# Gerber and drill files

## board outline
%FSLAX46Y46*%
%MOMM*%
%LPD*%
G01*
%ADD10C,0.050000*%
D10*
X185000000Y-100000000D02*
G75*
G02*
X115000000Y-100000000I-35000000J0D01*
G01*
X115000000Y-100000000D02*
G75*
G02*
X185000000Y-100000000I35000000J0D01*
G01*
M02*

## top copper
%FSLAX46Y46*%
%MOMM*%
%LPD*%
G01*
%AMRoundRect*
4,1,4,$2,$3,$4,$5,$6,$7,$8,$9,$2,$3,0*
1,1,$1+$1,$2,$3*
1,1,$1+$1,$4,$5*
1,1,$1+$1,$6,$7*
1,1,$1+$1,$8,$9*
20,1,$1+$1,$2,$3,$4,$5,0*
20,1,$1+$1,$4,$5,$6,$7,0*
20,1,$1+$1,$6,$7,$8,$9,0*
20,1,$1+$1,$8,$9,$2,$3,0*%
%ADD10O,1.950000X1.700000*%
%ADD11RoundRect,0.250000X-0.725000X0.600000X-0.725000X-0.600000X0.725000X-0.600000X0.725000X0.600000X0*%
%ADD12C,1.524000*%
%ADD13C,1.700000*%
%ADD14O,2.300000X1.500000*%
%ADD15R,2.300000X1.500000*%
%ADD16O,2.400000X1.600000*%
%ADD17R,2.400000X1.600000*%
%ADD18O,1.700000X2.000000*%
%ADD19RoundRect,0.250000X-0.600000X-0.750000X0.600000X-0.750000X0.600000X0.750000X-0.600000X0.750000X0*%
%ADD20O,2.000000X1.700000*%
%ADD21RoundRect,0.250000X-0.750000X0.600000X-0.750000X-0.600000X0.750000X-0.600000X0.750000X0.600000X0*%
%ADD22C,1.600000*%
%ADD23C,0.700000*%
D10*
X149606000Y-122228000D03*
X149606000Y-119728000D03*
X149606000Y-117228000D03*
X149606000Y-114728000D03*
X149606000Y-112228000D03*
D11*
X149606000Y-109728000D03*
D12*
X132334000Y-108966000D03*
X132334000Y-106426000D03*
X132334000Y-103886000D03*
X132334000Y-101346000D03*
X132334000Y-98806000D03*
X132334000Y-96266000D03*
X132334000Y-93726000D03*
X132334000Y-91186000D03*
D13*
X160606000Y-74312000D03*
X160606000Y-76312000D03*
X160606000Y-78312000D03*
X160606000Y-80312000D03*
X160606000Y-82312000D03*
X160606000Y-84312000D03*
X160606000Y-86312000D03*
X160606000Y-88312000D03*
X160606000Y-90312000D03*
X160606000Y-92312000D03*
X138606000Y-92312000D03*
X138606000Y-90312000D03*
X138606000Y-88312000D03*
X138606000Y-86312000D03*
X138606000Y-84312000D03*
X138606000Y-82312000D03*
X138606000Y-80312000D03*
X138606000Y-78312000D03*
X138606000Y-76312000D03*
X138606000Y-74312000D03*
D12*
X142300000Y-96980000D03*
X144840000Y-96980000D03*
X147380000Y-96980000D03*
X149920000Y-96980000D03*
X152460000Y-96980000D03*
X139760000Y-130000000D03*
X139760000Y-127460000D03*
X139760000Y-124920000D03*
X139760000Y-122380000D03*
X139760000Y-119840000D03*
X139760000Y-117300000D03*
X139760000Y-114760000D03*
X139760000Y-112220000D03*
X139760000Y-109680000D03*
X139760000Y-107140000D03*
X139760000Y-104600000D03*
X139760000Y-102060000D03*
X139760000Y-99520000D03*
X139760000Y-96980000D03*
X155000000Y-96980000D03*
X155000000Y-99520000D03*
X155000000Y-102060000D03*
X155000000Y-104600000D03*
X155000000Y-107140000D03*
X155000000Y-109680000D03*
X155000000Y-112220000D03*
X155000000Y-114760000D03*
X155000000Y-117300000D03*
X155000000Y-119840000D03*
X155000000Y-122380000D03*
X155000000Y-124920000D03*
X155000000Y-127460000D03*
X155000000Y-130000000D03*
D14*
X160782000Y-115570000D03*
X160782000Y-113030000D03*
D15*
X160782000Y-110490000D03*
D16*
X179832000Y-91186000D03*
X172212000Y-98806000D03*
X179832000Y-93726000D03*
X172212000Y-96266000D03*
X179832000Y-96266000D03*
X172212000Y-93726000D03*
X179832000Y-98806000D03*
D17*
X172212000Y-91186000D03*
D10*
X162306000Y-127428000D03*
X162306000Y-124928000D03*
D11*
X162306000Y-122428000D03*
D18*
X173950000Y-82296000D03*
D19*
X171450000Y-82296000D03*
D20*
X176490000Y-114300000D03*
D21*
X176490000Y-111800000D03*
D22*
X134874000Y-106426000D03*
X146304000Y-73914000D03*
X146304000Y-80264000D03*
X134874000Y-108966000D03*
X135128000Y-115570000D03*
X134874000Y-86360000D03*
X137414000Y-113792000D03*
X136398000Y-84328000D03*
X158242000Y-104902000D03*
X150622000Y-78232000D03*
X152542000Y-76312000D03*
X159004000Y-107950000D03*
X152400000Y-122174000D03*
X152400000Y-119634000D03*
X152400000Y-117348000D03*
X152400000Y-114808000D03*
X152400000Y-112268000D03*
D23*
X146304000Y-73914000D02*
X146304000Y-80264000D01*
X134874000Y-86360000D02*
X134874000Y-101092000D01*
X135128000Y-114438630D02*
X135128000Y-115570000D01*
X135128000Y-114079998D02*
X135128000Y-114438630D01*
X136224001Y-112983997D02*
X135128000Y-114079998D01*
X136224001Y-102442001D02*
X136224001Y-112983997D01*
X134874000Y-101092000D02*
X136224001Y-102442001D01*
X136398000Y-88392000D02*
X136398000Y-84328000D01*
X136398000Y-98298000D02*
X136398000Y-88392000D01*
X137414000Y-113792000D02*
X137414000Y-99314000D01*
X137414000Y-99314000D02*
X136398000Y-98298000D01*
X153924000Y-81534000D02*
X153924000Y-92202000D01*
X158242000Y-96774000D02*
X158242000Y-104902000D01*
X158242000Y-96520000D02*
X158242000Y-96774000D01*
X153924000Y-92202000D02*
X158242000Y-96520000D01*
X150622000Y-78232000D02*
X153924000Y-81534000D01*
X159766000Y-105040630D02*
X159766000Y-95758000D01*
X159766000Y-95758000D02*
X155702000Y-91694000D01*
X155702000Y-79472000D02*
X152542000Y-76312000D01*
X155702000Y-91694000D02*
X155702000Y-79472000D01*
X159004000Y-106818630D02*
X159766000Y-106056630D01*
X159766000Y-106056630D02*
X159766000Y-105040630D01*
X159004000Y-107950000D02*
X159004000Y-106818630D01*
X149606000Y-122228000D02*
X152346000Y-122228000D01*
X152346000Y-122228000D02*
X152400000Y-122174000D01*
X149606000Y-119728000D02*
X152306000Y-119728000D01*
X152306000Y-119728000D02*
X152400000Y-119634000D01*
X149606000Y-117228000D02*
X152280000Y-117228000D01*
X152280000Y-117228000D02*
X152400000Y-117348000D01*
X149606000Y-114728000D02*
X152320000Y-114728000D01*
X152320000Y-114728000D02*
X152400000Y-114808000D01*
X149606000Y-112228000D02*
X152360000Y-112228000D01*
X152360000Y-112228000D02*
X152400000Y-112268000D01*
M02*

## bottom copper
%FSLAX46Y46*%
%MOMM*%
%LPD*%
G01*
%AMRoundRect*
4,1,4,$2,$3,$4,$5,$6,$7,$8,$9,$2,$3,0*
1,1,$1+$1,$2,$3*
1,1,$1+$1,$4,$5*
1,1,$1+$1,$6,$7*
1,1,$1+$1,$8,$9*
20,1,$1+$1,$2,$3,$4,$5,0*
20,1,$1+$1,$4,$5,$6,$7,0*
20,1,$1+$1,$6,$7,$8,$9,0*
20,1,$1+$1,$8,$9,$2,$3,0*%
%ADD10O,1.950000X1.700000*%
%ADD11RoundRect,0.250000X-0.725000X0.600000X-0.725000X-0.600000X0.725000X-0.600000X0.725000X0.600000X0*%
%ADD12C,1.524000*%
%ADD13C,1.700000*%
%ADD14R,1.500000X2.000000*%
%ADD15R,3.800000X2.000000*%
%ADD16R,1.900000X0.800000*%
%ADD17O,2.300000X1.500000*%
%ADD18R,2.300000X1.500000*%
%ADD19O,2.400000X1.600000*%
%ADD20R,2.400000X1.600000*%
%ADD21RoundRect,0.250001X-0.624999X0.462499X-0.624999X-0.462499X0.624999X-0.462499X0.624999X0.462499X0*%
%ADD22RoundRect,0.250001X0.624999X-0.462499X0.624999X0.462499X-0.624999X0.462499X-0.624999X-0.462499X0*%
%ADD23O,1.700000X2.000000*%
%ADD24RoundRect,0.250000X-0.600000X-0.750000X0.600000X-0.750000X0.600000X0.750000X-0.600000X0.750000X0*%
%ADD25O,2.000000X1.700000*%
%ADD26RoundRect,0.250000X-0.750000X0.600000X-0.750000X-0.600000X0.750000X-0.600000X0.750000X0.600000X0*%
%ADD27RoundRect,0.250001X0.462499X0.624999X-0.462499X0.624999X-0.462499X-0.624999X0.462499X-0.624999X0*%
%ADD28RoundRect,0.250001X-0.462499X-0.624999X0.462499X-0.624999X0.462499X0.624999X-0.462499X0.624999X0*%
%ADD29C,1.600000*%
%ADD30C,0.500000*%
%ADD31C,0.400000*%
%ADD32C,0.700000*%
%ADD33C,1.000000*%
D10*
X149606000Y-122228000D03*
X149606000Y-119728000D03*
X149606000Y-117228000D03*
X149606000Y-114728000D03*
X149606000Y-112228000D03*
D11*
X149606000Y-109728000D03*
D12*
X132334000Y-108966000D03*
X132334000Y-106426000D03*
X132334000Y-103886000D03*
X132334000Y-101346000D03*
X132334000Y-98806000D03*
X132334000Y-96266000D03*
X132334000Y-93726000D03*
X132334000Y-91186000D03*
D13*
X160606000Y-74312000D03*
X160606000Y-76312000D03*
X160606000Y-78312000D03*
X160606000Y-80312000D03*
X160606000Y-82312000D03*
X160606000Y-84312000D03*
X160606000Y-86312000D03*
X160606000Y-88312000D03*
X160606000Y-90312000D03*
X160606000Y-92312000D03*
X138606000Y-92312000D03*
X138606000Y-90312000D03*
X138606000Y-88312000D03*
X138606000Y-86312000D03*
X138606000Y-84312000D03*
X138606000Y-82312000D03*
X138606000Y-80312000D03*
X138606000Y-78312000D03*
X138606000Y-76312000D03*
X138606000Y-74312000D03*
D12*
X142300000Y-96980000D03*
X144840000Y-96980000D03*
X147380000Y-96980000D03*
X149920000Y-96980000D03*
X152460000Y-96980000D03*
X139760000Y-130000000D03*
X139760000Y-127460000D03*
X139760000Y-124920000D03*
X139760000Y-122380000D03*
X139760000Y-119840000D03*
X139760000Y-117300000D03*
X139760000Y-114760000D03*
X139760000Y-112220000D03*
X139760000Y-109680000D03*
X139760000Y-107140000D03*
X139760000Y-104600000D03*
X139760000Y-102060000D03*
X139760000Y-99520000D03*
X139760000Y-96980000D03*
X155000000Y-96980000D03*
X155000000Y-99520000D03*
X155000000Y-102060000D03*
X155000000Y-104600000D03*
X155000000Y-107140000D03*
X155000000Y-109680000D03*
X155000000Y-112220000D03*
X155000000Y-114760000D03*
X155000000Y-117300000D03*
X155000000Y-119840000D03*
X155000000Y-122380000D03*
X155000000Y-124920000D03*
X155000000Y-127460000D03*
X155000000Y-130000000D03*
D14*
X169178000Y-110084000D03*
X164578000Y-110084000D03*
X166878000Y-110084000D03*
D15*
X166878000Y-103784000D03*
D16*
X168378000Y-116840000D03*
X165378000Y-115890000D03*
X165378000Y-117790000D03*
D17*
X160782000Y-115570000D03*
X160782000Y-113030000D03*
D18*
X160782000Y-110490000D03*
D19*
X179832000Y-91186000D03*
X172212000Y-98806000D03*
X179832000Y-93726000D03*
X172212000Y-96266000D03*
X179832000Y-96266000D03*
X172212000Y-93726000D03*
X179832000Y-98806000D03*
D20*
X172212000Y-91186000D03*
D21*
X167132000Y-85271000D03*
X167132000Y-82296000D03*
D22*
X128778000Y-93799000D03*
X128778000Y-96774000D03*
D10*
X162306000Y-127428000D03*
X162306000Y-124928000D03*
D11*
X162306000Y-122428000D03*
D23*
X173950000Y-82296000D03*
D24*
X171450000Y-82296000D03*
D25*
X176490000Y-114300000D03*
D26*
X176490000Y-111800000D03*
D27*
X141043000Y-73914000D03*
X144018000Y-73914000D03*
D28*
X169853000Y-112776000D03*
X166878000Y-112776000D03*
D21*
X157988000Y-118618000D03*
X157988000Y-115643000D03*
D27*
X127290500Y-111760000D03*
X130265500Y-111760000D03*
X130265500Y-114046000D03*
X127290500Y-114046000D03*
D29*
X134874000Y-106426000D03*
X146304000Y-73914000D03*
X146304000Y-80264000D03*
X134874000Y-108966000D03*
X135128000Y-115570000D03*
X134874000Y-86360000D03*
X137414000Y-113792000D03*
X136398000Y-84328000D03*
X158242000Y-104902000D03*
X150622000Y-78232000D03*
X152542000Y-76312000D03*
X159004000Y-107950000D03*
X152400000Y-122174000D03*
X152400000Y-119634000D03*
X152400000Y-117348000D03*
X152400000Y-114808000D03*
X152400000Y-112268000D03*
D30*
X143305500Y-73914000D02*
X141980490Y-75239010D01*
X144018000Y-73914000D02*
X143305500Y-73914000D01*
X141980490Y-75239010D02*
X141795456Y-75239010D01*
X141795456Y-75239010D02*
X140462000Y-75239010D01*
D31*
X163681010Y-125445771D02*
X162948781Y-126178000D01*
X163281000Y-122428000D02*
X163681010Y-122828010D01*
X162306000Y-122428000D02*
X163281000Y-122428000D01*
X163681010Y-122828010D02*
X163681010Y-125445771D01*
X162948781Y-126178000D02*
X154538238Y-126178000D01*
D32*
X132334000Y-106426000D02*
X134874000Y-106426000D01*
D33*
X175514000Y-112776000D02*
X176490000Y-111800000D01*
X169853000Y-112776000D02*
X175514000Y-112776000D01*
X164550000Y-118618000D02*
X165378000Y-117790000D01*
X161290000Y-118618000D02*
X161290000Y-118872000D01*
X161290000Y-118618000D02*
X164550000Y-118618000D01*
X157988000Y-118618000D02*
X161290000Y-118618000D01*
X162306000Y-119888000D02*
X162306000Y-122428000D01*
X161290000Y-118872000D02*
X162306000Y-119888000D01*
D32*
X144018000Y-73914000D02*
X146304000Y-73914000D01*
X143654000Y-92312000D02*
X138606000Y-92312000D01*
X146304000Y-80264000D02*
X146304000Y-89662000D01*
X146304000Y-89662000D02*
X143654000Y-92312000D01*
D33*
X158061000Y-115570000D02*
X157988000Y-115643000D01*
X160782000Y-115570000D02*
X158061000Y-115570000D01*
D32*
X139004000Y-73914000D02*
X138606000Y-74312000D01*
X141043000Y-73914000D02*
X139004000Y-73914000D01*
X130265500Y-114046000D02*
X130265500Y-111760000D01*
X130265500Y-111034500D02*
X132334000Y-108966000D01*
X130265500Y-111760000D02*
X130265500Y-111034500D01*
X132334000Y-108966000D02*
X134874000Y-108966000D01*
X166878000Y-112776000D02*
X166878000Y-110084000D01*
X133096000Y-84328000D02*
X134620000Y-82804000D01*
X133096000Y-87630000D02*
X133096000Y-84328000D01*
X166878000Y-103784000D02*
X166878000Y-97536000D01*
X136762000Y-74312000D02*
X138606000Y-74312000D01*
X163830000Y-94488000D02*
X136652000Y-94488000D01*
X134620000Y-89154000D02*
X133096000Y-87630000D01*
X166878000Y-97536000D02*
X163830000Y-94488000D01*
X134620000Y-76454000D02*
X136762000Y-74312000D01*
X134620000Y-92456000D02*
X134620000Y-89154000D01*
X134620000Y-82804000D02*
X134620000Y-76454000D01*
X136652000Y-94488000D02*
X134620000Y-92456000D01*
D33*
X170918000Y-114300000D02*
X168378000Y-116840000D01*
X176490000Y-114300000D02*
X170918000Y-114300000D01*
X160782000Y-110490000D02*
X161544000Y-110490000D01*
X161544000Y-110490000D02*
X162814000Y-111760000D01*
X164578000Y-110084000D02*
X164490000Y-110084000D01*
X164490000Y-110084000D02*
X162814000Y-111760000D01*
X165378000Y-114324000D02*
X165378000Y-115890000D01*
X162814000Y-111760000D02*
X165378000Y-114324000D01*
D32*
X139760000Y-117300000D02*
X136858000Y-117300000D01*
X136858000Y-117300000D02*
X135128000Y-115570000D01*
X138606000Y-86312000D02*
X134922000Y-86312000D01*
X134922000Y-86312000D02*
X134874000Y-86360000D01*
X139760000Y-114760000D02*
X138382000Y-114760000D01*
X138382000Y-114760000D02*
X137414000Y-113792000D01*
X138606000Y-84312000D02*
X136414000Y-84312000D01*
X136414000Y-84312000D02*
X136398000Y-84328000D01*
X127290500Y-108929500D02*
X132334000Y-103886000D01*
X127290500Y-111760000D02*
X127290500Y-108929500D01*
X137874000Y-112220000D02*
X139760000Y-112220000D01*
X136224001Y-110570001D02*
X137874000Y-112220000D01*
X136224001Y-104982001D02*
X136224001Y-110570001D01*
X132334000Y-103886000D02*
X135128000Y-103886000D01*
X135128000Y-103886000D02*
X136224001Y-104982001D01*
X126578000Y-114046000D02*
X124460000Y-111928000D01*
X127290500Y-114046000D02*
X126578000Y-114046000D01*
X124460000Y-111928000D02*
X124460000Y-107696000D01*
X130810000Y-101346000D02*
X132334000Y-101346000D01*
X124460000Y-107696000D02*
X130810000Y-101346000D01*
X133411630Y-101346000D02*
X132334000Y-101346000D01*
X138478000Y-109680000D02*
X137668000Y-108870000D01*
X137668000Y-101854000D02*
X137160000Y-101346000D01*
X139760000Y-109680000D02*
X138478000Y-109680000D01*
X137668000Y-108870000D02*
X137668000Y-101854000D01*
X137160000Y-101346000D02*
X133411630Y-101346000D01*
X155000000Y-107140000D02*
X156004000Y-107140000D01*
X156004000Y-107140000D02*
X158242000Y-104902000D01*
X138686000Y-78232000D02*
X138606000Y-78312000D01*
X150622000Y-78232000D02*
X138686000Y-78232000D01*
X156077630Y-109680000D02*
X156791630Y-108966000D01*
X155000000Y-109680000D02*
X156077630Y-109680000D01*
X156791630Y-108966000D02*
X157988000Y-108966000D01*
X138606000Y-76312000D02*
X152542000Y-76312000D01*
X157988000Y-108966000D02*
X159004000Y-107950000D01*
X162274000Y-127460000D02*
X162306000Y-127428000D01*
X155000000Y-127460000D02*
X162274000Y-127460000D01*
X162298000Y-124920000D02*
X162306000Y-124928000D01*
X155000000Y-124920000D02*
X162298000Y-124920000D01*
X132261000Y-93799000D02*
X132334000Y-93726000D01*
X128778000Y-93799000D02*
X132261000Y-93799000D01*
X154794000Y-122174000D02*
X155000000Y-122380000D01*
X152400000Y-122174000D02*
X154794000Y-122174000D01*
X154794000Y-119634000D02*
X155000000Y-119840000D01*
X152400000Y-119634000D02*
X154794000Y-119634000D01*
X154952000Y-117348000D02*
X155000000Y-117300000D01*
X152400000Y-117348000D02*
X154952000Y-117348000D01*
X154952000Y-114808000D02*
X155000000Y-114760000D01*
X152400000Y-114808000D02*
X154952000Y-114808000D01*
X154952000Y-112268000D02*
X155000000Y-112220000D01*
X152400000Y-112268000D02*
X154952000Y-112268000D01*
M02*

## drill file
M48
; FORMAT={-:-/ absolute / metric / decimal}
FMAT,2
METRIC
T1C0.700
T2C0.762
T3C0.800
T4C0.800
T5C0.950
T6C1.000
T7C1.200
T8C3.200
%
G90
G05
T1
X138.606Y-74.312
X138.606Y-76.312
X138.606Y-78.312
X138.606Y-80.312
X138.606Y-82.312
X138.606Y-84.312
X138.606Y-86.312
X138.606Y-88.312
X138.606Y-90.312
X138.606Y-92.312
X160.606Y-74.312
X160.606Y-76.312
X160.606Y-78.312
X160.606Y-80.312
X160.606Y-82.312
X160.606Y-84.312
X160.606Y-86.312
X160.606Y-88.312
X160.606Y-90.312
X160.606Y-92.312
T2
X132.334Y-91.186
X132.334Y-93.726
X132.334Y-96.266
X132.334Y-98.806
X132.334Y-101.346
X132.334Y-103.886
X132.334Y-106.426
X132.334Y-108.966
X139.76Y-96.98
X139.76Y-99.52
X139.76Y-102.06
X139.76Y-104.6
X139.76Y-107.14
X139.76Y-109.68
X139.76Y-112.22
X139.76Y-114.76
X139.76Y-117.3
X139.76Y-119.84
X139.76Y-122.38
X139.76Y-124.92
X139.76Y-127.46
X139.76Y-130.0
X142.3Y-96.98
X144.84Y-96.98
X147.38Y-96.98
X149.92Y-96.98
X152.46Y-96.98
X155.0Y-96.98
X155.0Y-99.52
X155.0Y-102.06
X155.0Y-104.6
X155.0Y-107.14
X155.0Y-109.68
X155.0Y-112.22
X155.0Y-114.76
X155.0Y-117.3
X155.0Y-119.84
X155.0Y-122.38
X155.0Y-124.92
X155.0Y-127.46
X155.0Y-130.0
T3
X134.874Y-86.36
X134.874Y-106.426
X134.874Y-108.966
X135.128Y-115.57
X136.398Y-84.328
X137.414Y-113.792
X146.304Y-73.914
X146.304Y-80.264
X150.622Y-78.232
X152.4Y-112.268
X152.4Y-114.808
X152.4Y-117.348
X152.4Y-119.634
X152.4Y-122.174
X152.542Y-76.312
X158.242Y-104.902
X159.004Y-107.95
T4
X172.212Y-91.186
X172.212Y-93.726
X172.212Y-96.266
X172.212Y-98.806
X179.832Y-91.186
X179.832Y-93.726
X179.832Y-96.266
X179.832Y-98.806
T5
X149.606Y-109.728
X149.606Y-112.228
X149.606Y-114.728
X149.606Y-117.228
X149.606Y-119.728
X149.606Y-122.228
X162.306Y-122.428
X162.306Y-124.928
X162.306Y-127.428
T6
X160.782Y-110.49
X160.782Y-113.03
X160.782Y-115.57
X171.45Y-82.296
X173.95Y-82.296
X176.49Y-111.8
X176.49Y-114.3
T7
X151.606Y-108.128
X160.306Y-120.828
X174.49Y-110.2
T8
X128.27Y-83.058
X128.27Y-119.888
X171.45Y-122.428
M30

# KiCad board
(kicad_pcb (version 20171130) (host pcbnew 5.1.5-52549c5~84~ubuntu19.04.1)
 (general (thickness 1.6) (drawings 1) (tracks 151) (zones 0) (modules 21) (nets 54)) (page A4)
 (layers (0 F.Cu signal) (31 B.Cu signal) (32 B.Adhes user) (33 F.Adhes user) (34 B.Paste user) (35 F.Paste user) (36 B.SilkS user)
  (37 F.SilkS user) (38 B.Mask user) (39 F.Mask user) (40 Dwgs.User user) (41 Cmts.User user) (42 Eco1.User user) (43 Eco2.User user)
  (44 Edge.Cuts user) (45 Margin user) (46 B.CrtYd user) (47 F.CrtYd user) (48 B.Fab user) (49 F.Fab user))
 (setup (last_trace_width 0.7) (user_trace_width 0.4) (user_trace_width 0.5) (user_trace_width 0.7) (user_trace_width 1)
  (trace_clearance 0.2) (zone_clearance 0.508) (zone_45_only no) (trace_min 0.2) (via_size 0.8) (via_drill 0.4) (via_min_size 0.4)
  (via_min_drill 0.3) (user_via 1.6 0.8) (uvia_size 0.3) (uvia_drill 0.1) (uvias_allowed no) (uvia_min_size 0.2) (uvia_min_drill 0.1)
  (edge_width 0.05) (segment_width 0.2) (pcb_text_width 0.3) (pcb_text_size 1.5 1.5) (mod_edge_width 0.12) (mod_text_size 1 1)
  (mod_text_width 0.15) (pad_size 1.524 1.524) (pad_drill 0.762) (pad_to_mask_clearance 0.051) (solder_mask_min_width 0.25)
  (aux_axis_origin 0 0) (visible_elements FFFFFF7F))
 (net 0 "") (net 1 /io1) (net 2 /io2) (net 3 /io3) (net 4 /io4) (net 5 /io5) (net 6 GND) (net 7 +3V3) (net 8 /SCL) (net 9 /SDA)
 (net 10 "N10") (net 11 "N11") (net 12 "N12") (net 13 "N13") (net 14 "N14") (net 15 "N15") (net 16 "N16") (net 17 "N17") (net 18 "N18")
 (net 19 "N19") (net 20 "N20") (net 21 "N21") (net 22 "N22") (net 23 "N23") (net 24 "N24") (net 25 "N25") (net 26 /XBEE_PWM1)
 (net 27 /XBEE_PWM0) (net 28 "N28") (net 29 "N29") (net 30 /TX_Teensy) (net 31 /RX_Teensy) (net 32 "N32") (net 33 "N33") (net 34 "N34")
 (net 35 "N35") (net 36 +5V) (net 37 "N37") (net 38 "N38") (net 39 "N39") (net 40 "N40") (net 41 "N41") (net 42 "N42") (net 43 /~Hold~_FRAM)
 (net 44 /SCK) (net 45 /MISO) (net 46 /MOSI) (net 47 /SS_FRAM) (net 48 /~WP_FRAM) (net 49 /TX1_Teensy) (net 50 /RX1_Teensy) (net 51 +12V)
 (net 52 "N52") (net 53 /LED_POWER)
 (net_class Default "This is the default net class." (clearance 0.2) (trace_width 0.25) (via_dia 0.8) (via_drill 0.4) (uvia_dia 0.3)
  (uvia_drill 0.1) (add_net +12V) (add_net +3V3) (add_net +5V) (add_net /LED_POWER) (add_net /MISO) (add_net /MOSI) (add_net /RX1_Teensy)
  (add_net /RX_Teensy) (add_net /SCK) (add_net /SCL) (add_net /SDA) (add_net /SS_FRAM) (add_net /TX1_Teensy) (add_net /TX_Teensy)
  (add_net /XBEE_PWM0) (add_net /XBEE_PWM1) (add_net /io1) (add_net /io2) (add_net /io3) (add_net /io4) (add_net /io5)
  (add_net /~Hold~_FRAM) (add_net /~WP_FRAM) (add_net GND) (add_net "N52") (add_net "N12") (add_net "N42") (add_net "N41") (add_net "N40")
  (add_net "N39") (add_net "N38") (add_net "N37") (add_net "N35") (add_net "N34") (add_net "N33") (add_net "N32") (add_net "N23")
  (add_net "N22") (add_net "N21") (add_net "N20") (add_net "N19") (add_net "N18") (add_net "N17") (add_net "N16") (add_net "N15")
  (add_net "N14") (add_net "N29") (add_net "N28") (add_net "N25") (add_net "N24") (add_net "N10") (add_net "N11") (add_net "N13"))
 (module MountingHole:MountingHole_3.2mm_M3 (layer F.Cu) (at 171.45 122.428)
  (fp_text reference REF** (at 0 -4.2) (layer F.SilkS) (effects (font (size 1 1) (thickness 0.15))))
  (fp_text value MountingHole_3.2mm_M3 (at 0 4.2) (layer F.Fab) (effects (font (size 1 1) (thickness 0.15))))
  (pad 1 np_thru_hole circle (at 0 0) (size 3.2 3.2) (drill 3.2) (layers *.Cu *.Mask)))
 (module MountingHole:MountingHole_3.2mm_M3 (layer F.Cu) (at 128.27 119.888)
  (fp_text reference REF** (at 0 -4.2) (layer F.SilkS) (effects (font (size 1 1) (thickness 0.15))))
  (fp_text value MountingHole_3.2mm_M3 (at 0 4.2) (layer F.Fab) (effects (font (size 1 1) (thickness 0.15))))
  (pad 1 np_thru_hole circle (at 0 0) (size 3.2 3.2) (drill 3.2) (layers *.Cu *.Mask)))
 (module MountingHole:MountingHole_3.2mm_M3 (layer F.Cu) (at 128.27 83.058)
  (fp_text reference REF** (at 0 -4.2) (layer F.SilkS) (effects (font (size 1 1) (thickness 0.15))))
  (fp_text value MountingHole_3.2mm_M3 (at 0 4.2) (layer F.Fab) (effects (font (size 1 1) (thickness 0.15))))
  (pad 1 np_thru_hole circle (at 0 0) (size 3.2 3.2) (drill 3.2) (layers *.Cu *.Mask)))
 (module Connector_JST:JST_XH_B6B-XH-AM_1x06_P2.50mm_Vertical (layer B.Cu) (at 149.606 109.728 270)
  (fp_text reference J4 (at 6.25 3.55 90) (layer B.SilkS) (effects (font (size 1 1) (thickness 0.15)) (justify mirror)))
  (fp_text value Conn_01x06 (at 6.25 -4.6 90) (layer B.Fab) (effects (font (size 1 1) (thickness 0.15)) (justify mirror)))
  (pad "" np_thru_hole circle (at -1.6 -2 270) (size 1.2 1.2) (drill 1.2) (layers *.Cu *.Mask))
  (pad 6 thru_hole oval (at 12.5 0 270) (size 1.7 1.95) (drill 0.95) (layers *.Cu *.Mask) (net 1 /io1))
  (pad 5 thru_hole oval (at 10 0 270) (size 1.7 1.95) (drill 0.95) (layers *.Cu *.Mask) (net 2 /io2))
  (pad 4 thru_hole oval (at 7.5 0 270) (size 1.7 1.95) (drill 0.95) (layers *.Cu *.Mask) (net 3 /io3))
  (pad 3 thru_hole oval (at 5 0 270) (size 1.7 1.95) (drill 0.95) (layers *.Cu *.Mask) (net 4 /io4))
  (pad 2 thru_hole oval (at 2.5 0 270) (size 1.7 1.95) (drill 0.95) (layers *.Cu *.Mask) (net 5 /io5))
  (pad 1 thru_hole roundrect (at 0 0 270) (size 1.7 1.95) (drill 0.95) (layers *.Cu *.Mask) (roundrect_rratio 0.147059) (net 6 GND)))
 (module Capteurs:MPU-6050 (layer F.Cu) (at 132.334 108.966 180)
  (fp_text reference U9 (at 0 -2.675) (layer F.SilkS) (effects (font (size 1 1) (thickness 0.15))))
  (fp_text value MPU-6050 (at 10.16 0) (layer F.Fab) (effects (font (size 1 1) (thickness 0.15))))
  (pad 1 thru_hole circle (at 0 0 180) (size 1.524 1.524) (drill 0.762) (layers *.Cu *.Mask) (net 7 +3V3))
  (pad 2 thru_hole circle (at 0 2.54 180) (size 1.524 1.524) (drill 0.762) (layers *.Cu *.Mask) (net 6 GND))
  (pad 3 thru_hole circle (at 0 5.08 180) (size 1.524 1.524) (drill 0.762) (layers *.Cu *.Mask) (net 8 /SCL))
  (pad 4 thru_hole circle (at 0 7.62 180) (size 1.524 1.524) (drill 0.762) (layers *.Cu *.Mask) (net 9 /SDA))
  (pad 5 thru_hole circle (at 0 10.16 180) (size 1.524 1.524) (drill 0.762) (layers *.Cu *.Mask) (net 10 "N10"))
  (pad 6 thru_hole circle (at 0 12.7 180) (size 1.524 1.524) (drill 0.762) (layers *.Cu *.Mask) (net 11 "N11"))
  (pad 7 thru_hole circle (at 0 15.24 180) (size 1.524 1.524) (drill 0.762) (layers *.Cu *.Mask) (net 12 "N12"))
  (pad 8 thru_hole circle (at 0 17.78 180) (size 1.524 1.524) (drill 0.762) (layers *.Cu *.Mask) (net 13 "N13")))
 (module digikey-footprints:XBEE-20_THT (layer F.Cu) (at 149.606 83.312)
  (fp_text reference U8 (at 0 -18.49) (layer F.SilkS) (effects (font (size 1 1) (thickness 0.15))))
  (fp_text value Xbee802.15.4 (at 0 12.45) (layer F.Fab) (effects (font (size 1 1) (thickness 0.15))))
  (pad 20 thru_hole circle (at 11 -9) (size 1.7 1.7) (drill 0.7) (layers *.Cu *.Mask) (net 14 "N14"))
  (pad 19 thru_hole circle (at 11 -7) (size 1.7 1.7) (drill 0.7) (layers *.Cu *.Mask) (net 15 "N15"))
  (pad 18 thru_hole circle (at 11 -5) (size 1.7 1.7) (drill 0.7) (layers *.Cu *.Mask) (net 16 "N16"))
  (pad 17 thru_hole circle (at 11 -3) (size 1.7 1.7) (drill 0.7) (layers *.Cu *.Mask) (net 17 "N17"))
  (pad 16 thru_hole circle (at 11 -1) (size 1.7 1.7) (drill 0.7) (layers *.Cu *.Mask) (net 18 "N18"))
  (pad 15 thru_hole circle (at 11 1) (size 1.7 1.7) (drill 0.7) (layers *.Cu *.Mask) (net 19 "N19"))
  (pad 14 thru_hole circle (at 11 3) (size 1.7 1.7) (drill 0.7) (layers *.Cu *.Mask) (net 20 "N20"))
  (pad 13 thru_hole circle (at 11 5) (size 1.7 1.7) (drill 0.7) (layers *.Cu *.Mask) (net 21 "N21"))
  (pad 12 thru_hole circle (at 11 7) (size 1.7 1.7) (drill 0.7) (layers *.Cu *.Mask) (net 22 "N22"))
  (pad 11 thru_hole circle (at 11 9) (size 1.7 1.7) (drill 0.7) (layers *.Cu *.Mask) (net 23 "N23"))
  (pad 10 thru_hole circle (at -11 9) (size 1.7 1.7) (drill 0.7) (layers *.Cu *.Mask) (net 6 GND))
  (pad 9 thru_hole circle (at -11 7) (size 1.7 1.7) (drill 0.7) (layers *.Cu *.Mask) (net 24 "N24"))
  (pad 8 thru_hole circle (at -11 5) (size 1.7 1.7) (drill 0.7) (layers *.Cu *.Mask) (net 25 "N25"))
  (pad 7 thru_hole circle (at -11 3) (size 1.7 1.7) (drill 0.7) (layers *.Cu *.Mask) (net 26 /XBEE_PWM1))
  (pad 6 thru_hole circle (at -11 1) (size 1.7 1.7) (drill 0.7) (layers *.Cu *.Mask) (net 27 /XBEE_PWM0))
  (pad 5 thru_hole circle (at -11 -1) (size 1.7 1.7) (drill 0.7) (layers *.Cu *.Mask) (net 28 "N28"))
  (pad 4 thru_hole circle (at -11 -3) (size 1.7 1.7) (drill 0.7) (layers *.Cu *.Mask) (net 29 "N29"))
  (pad 3 thru_hole circle (at -11 -5) (size 1.7 1.7) (drill 0.7) (layers *.Cu *.Mask) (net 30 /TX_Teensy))
  (pad 2 thru_hole circle (at -11 -7) (size 1.7 1.7) (drill 0.7) (layers *.Cu *.Mask) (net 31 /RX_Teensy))
  (pad 1 thru_hole circle (at -11 -9) (size 1.7 1.7) (drill 0.7) (layers *.Cu *.Mask) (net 7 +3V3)))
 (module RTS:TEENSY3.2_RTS (layer F.Cu) (at 155 130 180)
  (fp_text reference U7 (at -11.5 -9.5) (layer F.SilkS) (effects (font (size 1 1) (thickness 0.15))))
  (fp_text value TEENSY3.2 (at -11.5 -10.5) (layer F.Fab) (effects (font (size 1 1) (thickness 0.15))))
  (pad 33 thru_hole circle (at 12.7 33.02 180) (size 1.524 1.524) (drill 0.762) (layers *.Cu *.Mask) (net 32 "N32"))
  (pad 32 thru_hole circle (at 10.16 33.02 180) (size 1.524 1.524) (drill 0.762) (layers *.Cu *.Mask) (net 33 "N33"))
  (pad 31 thru_hole circle (at 7.62 33.02 180) (size 1.524 1.524) (drill 0.762) (layers *.Cu *.Mask) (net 6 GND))
  (pad 30 thru_hole circle (at 5.08 33.02 180) (size 1.524 1.524) (drill 0.762) (layers *.Cu *.Mask) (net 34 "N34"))
  (pad 29 thru_hole circle (at 2.54 33.02 180) (size 1.524 1.524) (drill 0.762) (layers *.Cu *.Mask) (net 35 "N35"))
  (pad 28 thru_hole circle (at 15.24 0 180) (size 1.524 1.524) (drill 0.762) (layers *.Cu *.Mask) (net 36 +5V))
  (pad 27 thru_hole circle (at 15.24 2.54 180) (size 1.524 1.524) (drill 0.762) (layers *.Cu *.Mask) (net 6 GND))
  (pad 26 thru_hole circle (at 15.24 5.08 180) (size 1.524 1.524) (drill 0.762) (layers *.Cu *.Mask) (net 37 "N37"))
  (pad 25 thru_hole circle (at 15.24 7.62 180) (size 1.524 1.524) (drill 0.762) (layers *.Cu *.Mask) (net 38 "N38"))
  (pad 24 thru_hole circle (at 15.24 10.16 180) (size 1.524 1.524) (drill 0.762) (layers *.Cu *.Mask) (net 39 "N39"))
  (pad 23 thru_hole circle (at 15.24 12.7 180) (size 1.524 1.524) (drill 0.762) (layers *.Cu *.Mask) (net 26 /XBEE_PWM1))
  (pad 22 thru_hole circle (at 15.24 15.24 180) (size 1.524 1.524) (drill 0.762) (layers *.Cu *.Mask) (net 27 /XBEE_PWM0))
  (pad 21 thru_hole circle (at 15.24 17.78 180) (size 1.524 1.524) (drill 0.762) (layers *.Cu *.Mask) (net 8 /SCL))
  (pad 20 thru_hole circle (at 15.24 20.32 180) (size 1.524 1.524) (drill 0.762) (layers *.Cu *.Mask) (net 9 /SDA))
  (pad 19 thru_hole circle (at 15.24 22.86 180) (size 1.524 1.524) (drill 0.762) (layers *.Cu *.Mask) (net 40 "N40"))
  (pad 18 thru_hole circle (at 15.24 25.4 180) (size 1.524 1.524) (drill 0.762) (layers *.Cu *.Mask) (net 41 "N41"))
  (pad 17 thru_hole circle (at 15.24 27.94 180) (size 1.524 1.524) (drill 0.762) (layers *.Cu *.Mask) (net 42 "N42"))
  (pad 16 thru_hole circle (at 15.24 30.48 180) (size 1.524 1.524) (drill 0.762) (layers *.Cu *.Mask) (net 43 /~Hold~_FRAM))
  (pad 15 thru_hole circle (at 15.24 33.02 180) (size 1.524 1.524) (drill 0.762) (layers *.Cu *.Mask) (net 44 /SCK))
  (pad 14 thru_hole circle (at 0 33.02 180) (size 1.524 1.524) (drill 0.762) (layers *.Cu *.Mask) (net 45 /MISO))
  (pad 13 thru_hole circle (at 0 30.48 180) (size 1.524 1.524) (drill 0.762) (layers *.Cu *.Mask) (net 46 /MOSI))
  (pad 12 thru_hole circle (at 0 27.94 180) (size 1.524 1.524) (drill 0.762) (layers *.Cu *.Mask) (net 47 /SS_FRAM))
  (pad 11 thru_hole circle (at 0 25.4 180) (size 1.524 1.524) (drill 0.762) (layers *.Cu *.Mask) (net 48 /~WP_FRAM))
  (pad 10 thru_hole circle (at 0 22.86 180) (size 1.524 1.524) (drill 0.762) (layers *.Cu *.Mask) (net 30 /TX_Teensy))
  (pad 9 thru_hole circle (at 0 20.32 180) (size 1.524 1.524) (drill 0.762) (layers *.Cu *.Mask) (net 31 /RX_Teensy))
  (pad 8 thru_hole circle (at 0 17.78 180) (size 1.524 1.524) (drill 0.762) (layers *.Cu *.Mask) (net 5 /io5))
  (pad 7 thru_hole circle (at 0 15.24 180) (size 1.524 1.524) (drill 0.762) (layers *.Cu *.Mask) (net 4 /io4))
  (pad 6 thru_hole circle (at 0 12.7 180) (size 1.524 1.524) (drill 0.762) (layers *.Cu *.Mask) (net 3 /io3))
  (pad 5 thru_hole circle (at 0 10.16 180) (size 1.524 1.524) (drill 0.762) (layers *.Cu *.Mask) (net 2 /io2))
  (pad 4 thru_hole circle (at 0 7.62 180) (size 1.524 1.524) (drill 0.762) (layers *.Cu *.Mask) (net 1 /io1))
  (pad 3 thru_hole circle (at 0 5.08 180) (size 1.524 1.524) (drill 0.762) (layers *.Cu *.Mask) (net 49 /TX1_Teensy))
  (pad 2 thru_hole circle (at 0 2.54 180) (size 1.524 1.524) (drill 0.762) (layers *.Cu *.Mask) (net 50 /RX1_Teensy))
  (pad 1 thru_hole circle (at 0 0 180) (size 1.524 1.524) (drill 0.762) (layers *.Cu *.Mask) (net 6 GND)))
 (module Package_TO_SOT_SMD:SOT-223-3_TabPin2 (layer B.Cu) (at 166.878 106.934 90)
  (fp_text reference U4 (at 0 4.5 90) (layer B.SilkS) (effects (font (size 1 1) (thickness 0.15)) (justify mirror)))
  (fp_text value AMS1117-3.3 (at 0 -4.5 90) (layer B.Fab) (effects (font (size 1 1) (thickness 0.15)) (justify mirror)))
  (pad 1 smd rect (at -3.15 2.3 90) (size 2 1.5) (layers B.Cu B.Paste B.Mask) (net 6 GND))
  (pad 3 smd rect (at -3.15 -2.3 90) (size 2 1.5) (layers B.Cu B.Paste B.Mask) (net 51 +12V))
  (pad 2 smd rect (at -3.15 0 90) (size 2 1.5) (layers B.Cu B.Paste B.Mask) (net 7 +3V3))
  (pad 2 smd rect (at 3.15 0 90) (size 2 3.8) (layers B.Cu B.Paste B.Mask) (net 7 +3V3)))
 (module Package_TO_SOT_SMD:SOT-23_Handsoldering (layer B.Cu) (at 166.878 116.84)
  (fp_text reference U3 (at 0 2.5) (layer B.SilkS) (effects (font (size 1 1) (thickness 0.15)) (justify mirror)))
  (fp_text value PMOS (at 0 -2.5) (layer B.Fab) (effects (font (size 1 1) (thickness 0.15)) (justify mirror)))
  (pad 3 smd rect (at 1.5 0) (size 1.9 0.8) (layers B.Cu B.Paste B.Mask) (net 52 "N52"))
  (pad 2 smd rect (at -1.5 -0.95) (size 1.9 0.8) (layers B.Cu B.Paste B.Mask) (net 51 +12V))
  (pad 1 smd rect (at -1.5 0.95) (size 1.9 0.8) (layers B.Cu B.Paste B.Mask) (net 6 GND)))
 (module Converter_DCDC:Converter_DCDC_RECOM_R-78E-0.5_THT (layer F.Cu) (at 160.782 110.49 270)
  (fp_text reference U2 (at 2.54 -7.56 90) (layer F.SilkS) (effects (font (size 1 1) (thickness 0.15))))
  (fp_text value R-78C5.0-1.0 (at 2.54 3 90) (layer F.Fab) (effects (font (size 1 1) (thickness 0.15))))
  (pad 3 thru_hole oval (at 5.08 0 270) (size 1.5 2.3) (drill 1) (layers *.Cu *.Mask) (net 36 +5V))
  (pad 2 thru_hole oval (at 2.54 0 270) (size 1.5 2.3) (drill 1) (layers *.Cu *.Mask) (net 6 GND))
  (pad 1 thru_hole rect (at 0 0 270) (size 1.5 2.3) (drill 1) (layers *.Cu *.Mask) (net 51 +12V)))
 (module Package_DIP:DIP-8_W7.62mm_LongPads (layer F.Cu) (at 172.212 91.186)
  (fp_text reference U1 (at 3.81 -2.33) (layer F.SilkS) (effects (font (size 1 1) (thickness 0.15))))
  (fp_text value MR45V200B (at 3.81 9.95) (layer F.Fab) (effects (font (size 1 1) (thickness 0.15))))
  (pad 8 thru_hole oval (at 7.62 0) (size 2.4 1.6) (drill 0.8) (layers *.Cu *.Mask) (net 7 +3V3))
  (pad 4 thru_hole oval (at 0 7.62) (size 2.4 1.6) (drill 0.8) (layers *.Cu *.Mask) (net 6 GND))
  (pad 7 thru_hole oval (at 7.62 2.54) (size 2.4 1.6) (drill 0.8) (layers *.Cu *.Mask) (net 43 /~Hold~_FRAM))
  (pad 3 thru_hole oval (at 0 5.08) (size 2.4 1.6) (drill 0.8) (layers *.Cu *.Mask) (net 48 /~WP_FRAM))
  (pad 6 thru_hole oval (at 7.62 5.08) (size 2.4 1.6) (drill 0.8) (layers *.Cu *.Mask) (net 44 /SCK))
  (pad 2 thru_hole oval (at 0 2.54) (size 2.4 1.6) (drill 0.8) (layers *.Cu *.Mask) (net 45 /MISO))
  (pad 5 thru_hole oval (at 7.62 7.62) (size 2.4 1.6) (drill 0.8) (layers *.Cu *.Mask) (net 46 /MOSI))
  (pad 1 thru_hole rect (at 0 0) (size 2.4 1.6) (drill 0.8) (layers *.Cu *.Mask) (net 47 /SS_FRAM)))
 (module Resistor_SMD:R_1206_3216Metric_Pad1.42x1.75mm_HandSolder (layer B.Cu) (at 167.132 83.7835 270)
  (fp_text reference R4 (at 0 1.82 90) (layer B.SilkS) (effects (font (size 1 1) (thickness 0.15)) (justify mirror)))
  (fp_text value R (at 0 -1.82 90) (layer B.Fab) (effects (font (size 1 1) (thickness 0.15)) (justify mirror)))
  (pad 2 smd roundrect (at 1.4875 0 270) (size 1.425 1.75) (layers B.Cu B.Paste B.Mask) (roundrect_rratio 0.175439) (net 36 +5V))
  (pad 1 smd roundrect (at -1.4875 0 270) (size 1.425 1.75) (layers B.Cu B.Paste B.Mask) (roundrect_rratio 0.175439) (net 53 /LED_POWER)))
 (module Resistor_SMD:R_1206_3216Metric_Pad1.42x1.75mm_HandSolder (layer B.Cu) (at 128.778 95.2865 90)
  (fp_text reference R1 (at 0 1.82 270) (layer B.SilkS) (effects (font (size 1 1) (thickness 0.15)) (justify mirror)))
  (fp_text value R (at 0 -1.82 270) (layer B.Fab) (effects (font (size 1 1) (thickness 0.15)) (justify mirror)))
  (pad 2 smd roundrect (at 1.4875 0 90) (size 1.425 1.75) (layers B.Cu B.Paste B.Mask) (roundrect_rratio 0.175439) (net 12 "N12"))
  (pad 1 smd roundrect (at -1.4875 0 90) (size 1.425 1.75) (layers B.Cu B.Paste B.Mask) (roundrect_rratio 0.175439) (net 6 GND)))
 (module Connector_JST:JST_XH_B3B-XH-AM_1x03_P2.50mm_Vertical (layer F.Cu) (at 162.306 122.428 270)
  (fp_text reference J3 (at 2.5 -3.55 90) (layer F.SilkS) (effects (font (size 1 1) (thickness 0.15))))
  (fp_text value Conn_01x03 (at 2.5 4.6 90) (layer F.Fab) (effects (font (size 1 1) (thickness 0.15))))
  (pad "" np_thru_hole circle (at -1.6 2 270) (size 1.2 1.2) (drill 1.2) (layers *.Cu *.Mask))
  (pad 3 thru_hole oval (at 5 0 270) (size 1.7 1.95) (drill 0.95) (layers *.Cu *.Mask) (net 50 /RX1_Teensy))
  (pad 2 thru_hole oval (at 2.5 0 270) (size 1.7 1.95) (drill 0.95) (layers *.Cu *.Mask) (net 49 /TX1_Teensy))
  (pad 1 thru_hole roundrect (at 0 0 270) (size 1.7 1.95) (drill 0.95) (layers *.Cu *.Mask) (roundrect_rratio 0.147059) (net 6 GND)))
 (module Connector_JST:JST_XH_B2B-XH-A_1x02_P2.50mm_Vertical (layer F.Cu) (at 171.45 82.296)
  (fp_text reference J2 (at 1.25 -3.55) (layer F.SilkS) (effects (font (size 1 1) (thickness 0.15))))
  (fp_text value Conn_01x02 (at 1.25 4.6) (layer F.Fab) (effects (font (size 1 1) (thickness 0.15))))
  (pad 2 thru_hole oval (at 2.5 0) (size 1.7 2) (drill 1) (layers *.Cu *.Mask) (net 6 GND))
  (pad 1 thru_hole roundrect (at 0 0) (size 1.7 2) (drill 1) (layers *.Cu *.Mask) (roundrect_rratio 0.147059) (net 53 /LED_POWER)))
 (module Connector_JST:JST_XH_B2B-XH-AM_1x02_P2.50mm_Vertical (layer F.Cu) (at 176.49 111.8 270)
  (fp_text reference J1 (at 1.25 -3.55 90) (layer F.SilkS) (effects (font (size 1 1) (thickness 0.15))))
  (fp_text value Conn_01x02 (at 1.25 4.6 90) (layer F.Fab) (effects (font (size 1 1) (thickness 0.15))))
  (pad "" np_thru_hole circle (at -1.6 2 270) (size 1.2 1.2) (drill 1.2) (layers *.Cu *.Mask))
  (pad 2 thru_hole oval (at 2.5 0 270) (size 1.7 2) (drill 1) (layers *.Cu *.Mask) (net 52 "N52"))
  (pad 1 thru_hole roundrect (at 0 0 270) (size 1.7 2) (drill 1) (layers *.Cu *.Mask) (roundrect_rratio 0.147059) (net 6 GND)))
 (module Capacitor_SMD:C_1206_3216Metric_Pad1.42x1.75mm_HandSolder (layer B.Cu) (at 142.5305 73.914 180)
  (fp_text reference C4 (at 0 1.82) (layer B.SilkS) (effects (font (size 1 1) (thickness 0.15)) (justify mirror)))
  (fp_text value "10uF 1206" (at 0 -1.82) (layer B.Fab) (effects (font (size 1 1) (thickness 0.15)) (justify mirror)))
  (pad 2 smd roundrect (at 1.4875 0 180) (size 1.425 1.75) (layers B.Cu B.Paste B.Mask) (roundrect_rratio 0.175439) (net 7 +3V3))
  (pad 1 smd roundrect (at -1.4875 0 180) (size 1.425 1.75) (layers B.Cu B.Paste B.Mask) (roundrect_rratio 0.175439) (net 6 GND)))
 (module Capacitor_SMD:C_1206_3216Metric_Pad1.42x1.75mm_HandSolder (layer B.Cu) (at 168.3655 112.776)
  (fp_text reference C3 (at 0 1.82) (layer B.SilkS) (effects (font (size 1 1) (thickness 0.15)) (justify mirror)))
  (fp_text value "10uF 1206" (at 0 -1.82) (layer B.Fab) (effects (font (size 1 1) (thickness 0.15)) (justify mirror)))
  (pad 2 smd roundrect (at 1.4875 0) (size 1.425 1.75) (layers B.Cu B.Paste B.Mask) (roundrect_rratio 0.175439) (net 6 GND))
  (pad 1 smd roundrect (at -1.4875 0) (size 1.425 1.75) (layers B.Cu B.Paste B.Mask) (roundrect_rratio 0.175439) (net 7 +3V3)))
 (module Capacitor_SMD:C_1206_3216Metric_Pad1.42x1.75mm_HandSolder (layer B.Cu) (at 157.988 117.1305 270)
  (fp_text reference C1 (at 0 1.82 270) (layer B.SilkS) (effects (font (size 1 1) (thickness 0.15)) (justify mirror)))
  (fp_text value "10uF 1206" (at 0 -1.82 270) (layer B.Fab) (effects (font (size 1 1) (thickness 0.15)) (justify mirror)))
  (pad 2 smd roundrect (at 1.4875 0 270) (size 1.425 1.75) (layers B.Cu B.Paste B.Mask) (roundrect_rratio 0.175439) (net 6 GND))
  (pad 1 smd roundrect (at -1.4875 0 270) (size 1.425 1.75) (layers B.Cu B.Paste B.Mask) (roundrect_rratio 0.175439) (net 36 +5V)))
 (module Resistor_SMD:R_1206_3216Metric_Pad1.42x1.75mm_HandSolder (layer B.Cu) (at 128.778 111.76 180)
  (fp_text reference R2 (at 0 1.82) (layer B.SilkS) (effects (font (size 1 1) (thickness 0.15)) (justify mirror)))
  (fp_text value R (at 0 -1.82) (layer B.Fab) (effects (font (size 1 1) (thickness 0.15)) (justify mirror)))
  (pad 2 smd roundrect (at 1.4875 0 180) (size 1.425 1.75) (layers B.Cu B.Paste B.Mask) (roundrect_rratio 0.175439) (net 8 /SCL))
  (pad 1 smd roundrect (at -1.4875 0 180) (size 1.425 1.75) (layers B.Cu B.Paste B.Mask) (roundrect_rratio 0.175439) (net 7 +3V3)))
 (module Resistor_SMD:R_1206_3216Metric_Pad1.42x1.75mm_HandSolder (layer B.Cu) (at 128.778 114.046 180)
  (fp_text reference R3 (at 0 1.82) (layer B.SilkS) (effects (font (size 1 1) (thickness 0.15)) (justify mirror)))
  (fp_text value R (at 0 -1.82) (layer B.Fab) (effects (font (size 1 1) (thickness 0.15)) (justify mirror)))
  (pad 1 smd roundrect (at -1.4875 0 180) (size 1.425 1.75) (layers B.Cu B.Paste B.Mask) (roundrect_rratio 0.175439) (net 7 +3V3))
  (pad 2 smd roundrect (at 1.4875 0 180) (size 1.425 1.75) (layers B.Cu B.Paste B.Mask) (roundrect_rratio 0.175439) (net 9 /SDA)))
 (gr_circle (center 150 100) (end 115 100) (layer Edge.Cuts) (width 0.05))
 (segment (start 143.3055 73.914) (end 141.98049 75.23901) (width 0.5) (layer B.Cu) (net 6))
 (segment (start 144.018 73.914) (end 143.3055 73.914) (width 0.5) (layer B.Cu) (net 6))
 (segment (start 141.98049 75.23901) (end 141.795456 75.23901) (width 0.5) (layer B.Cu) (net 6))
 (segment (start 141.795456 75.23901) (end 140.462 75.23901) (width 0.5) (layer B.Cu) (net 6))
 (segment (start 163.68101 125.445771) (end 162.948781 126.178) (width 0.4) (layer B.Cu) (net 6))
 (segment (start 163.281 122.428) (end 163.68101 122.82801) (width 0.4) (layer B.Cu) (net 6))
 (segment (start 162.306 122.428) (end 163.281 122.428) (width 0.4) (layer B.Cu) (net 6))
 (segment (start 163.68101 122.82801) (end 163.68101 125.445771) (width 0.4) (layer B.Cu) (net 6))
 (segment (start 162.948781 126.178) (end 154.538238 126.178) (width 0.4) (layer B.Cu) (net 6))
 (via (at 134.874 106.426) (size 1.6) (drill 0.8) (layers F.Cu B.Cu) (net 6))
 (segment (start 132.334 106.426) (end 134.874 106.426) (width 0.7) (layer B.Cu) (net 6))
 (segment (start 175.514 112.776) (end 176.49 111.8) (width 1) (layer B.Cu) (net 6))
 (segment (start 169.853 112.776) (end 175.514 112.776) (width 1) (layer B.Cu) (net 6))
 (segment (start 164.55 118.618) (end 165.378 117.79) (width 1) (layer B.Cu) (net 6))
 (segment (start 161.29 118.618) (end 161.29 118.872) (width 1) (layer B.Cu) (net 6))
 (segment (start 161.29 118.618) (end 164.55 118.618) (width 1) (layer B.Cu) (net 6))
 (segment (start 157.988 118.618) (end 161.29 118.618) (width 1) (layer B.Cu) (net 6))
 (segment (start 162.306 119.888) (end 162.306 122.428) (width 1) (layer B.Cu) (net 6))
 (segment (start 161.29 118.872) (end 162.306 119.888) (width 1) (layer B.Cu) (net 6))
 (via (at 146.304 73.914) (size 1.6) (drill 0.8) (layers F.Cu B.Cu) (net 6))
 (segment (start 144.018 73.914) (end 146.304 73.914) (width 0.7) (layer B.Cu) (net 6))
 (via (at 146.304 80.264) (size 1.6) (drill 0.8) (layers F.Cu B.Cu) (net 6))
 (segment (start 146.304 73.914) (end 146.304 80.264) (width 0.7) (layer F.Cu) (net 6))
 (segment (start 143.654 92.312) (end 138.606 92.312) (width 0.7) (layer B.Cu) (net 6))
 (segment (start 146.304 80.264) (end 146.304 89.662) (width 0.7) (layer B.Cu) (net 6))
 (segment (start 146.304 89.662) (end 143.654 92.312) (width 0.7) (layer B.Cu) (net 6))
 (segment (start 158.061 115.57) (end 157.988 115.643) (width 1) (layer B.Cu) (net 36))
 (segment (start 160.782 115.57) (end 158.061 115.57) (width 1) (layer B.Cu) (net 36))
 (segment (start 139.004 73.914) (end 138.606 74.312) (width 0.7) (layer B.Cu) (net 7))
 (segment (start 141.043 73.914) (end 139.004 73.914) (width 0.7) (layer B.Cu) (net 7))
 (segment (start 130.2655 114.046) (end 130.2655 111.76) (width 0.7) (layer B.Cu) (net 7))
 (segment (start 130.2655 111.0345) (end 132.334 108.966) (width 0.7) (layer B.Cu) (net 7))
 (segment (start 130.2655 111.76) (end 130.2655 111.0345) (width 0.7) (layer B.Cu) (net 7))
 (via (at 134.874 108.966) (size 1.6) (drill 0.8) (layers F.Cu B.Cu) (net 7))
 (segment (start 132.334 108.966) (end 134.874 108.966) (width 0.7) (layer B.Cu) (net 7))
 (segment (start 166.878 112.776) (end 166.878 110.084) (width 0.7) (layer B.Cu) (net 7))
 (segment (start 133.096 84.328) (end 134.62 82.804) (width 0.7) (layer B.Cu) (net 7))
 (segment (start 133.096 87.63) (end 133.096 84.328) (width 0.7) (layer B.Cu) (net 7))
 (segment (start 166.878 103.784) (end 166.878 97.536) (width 0.7) (layer B.Cu) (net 7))
 (segment (start 136.762 74.312) (end 138.606 74.312) (width 0.7) (layer B.Cu) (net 7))
 (segment (start 163.83 94.488) (end 136.652 94.488) (width 0.7) (layer B.Cu) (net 7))
 (segment (start 134.62 89.154) (end 133.096 87.63) (width 0.7) (layer B.Cu) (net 7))
 (segment (start 166.878 97.536) (end 163.83 94.488) (width 0.7) (layer B.Cu) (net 7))
 (segment (start 134.62 76.454) (end 136.762 74.312) (width 0.7) (layer B.Cu) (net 7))
 (segment (start 134.62 92.456) (end 134.62 89.154) (width 0.7) (layer B.Cu) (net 7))
 (segment (start 134.62 82.804) (end 134.62 76.454) (width 0.7) (layer B.Cu) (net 7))
 (segment (start 136.652 94.488) (end 134.62 92.456) (width 0.7) (layer B.Cu) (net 7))
 (segment (start 170.918 114.3) (end 168.378 116.84) (width 1) (layer B.Cu) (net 52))
 (segment (start 176.49 114.3) (end 170.918 114.3) (width 1) (layer B.Cu) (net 52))
 (segment (start 160.782 110.49) (end 161.544 110.49) (width 1) (layer B.Cu) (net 51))
 (segment (start 161.544 110.49) (end 162.814 111.76) (width 1) (layer B.Cu) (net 51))
 (segment (start 164.578 110.084) (end 164.49 110.084) (width 1) (layer B.Cu) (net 51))
 (segment (start 164.49 110.084) (end 162.814 111.76) (width 1) (layer B.Cu) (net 51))
 (segment (start 165.378 114.324) (end 165.378 115.89) (width 1) (layer B.Cu) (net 51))
 (segment (start 162.814 111.76) (end 165.378 114.324) (width 1) (layer B.Cu) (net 51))
 (via (at 135.128 115.57) (size 1.6) (drill 0.8) (layers F.Cu B.Cu) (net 26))
 (segment (start 139.76 117.3) (end 136.858 117.3) (width 0.7) (layer B.Cu) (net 26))
 (segment (start 136.858 117.3) (end 135.128 115.57) (width 0.7) (layer B.Cu) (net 26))
 (via (at 134.874 86.36) (size 1.6) (drill 0.8) (layers F.Cu B.Cu) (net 26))
 (segment (start 138.606 86.312) (end 134.922 86.312) (width 0.7) (layer B.Cu) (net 26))
 (segment (start 134.922 86.312) (end 134.874 86.36) (width 0.7) (layer B.Cu) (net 26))
 (segment (start 134.874 86.36) (end 134.874 101.092) (width 0.7) (layer F.Cu) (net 26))
 (segment (start 135.128 114.43863) (end 135.128 115.57) (width 0.7) (layer F.Cu) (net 26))
 (segment (start 135.128 114.079998) (end 135.128 114.43863) (width 0.7) (layer F.Cu) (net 26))
 (segment (start 136.224001 112.983997) (end 135.128 114.079998) (width 0.7) (layer F.Cu) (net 26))
 (segment (start 136.224001 102.442001) (end 136.224001 112.983997) (width 0.7) (layer F.Cu) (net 26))
 (segment (start 134.874 101.092) (end 136.224001 102.442001) (width 0.7) (layer F.Cu) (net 26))
 (via (at 137.414 113.792) (size 1.6) (drill 0.8) (layers F.Cu B.Cu) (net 27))
 (segment (start 139.76 114.76) (end 138.382 114.76) (width 0.7) (layer B.Cu) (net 27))
 (segment (start 138.382 114.76) (end 137.414 113.792) (width 0.7) (layer B.Cu) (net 27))
 (via (at 136.398 84.328) (size 1.6) (drill 0.8) (layers F.Cu B.Cu) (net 27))
 (segment (start 138.606 84.312) (end 136.414 84.312) (width 0.7) (layer B.Cu) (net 27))
 (segment (start 136.414 84.312) (end 136.398 84.328) (width 0.7) (layer B.Cu) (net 27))
 (segment (start 136.398 88.392) (end 136.398 84.328) (width 0.7) (layer F.Cu) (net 27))
 (segment (start 136.398 98.298) (end 136.398 88.392) (width 0.7) (layer F.Cu) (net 27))
 (segment (start 137.414 113.792) (end 137.414 99.314) (width 0.7) (layer F.Cu) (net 27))
 (segment (start 137.414 99.314) (end 136.398 98.298) (width 0.7) (layer F.Cu) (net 27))
 (segment (start 127.2905 108.9295) (end 132.334 103.886) (width 0.7) (layer B.Cu) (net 8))
 (segment (start 127.2905 111.76) (end 127.2905 108.9295) (width 0.7) (layer B.Cu) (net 8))
 (segment (start 137.874 112.22) (end 139.76 112.22) (width 0.7) (layer B.Cu) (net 8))
 (segment (start 136.224001 110.570001) (end 137.874 112.22) (width 0.7) (layer B.Cu) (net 8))
 (segment (start 136.224001 104.982001) (end 136.224001 110.570001) (width 0.7) (layer B.Cu) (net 8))
 (segment (start 132.334 103.886) (end 135.128 103.886) (width 0.7) (layer B.Cu) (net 8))
 (segment (start 135.128 103.886) (end 136.224001 104.982001) (width 0.7) (layer B.Cu) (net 8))
 (segment (start 126.578 114.046) (end 124.46 111.928) (width 0.7) (layer B.Cu) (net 9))
 (segment (start 127.2905 114.046) (end 126.578 114.046) (width 0.7) (layer B.Cu) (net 9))
 (segment (start 124.46 111.928) (end 124.46 107.696) (width 0.7) (layer B.Cu) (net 9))
 (segment (start 130.81 101.346) (end 132.334 101.346) (width 0.7) (layer B.Cu) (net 9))
 (segment (start 124.46 107.696) (end 130.81 101.346) (width 0.7) (layer B.Cu) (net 9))
 (segment (start 133.41163 101.346) (end 132.334 101.346) (width 0.7) (layer B.Cu) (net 9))
 (segment (start 138.478 109.68) (end 137.668 108.87) (width 0.7) (layer B.Cu) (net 9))
 (segment (start 137.668 101.854) (end 137.16 101.346) (width 0.7) (layer B.Cu) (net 9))
 (segment (start 139.76 109.68) (end 138.478 109.68) (width 0.7) (layer B.Cu) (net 9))
 (segment (start 137.668 108.87) (end 137.668 101.854) (width 0.7) (layer B.Cu) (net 9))
 (segment (start 137.16 101.346) (end 133.41163 101.346) (width 0.7) (layer B.Cu) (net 9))
 (via (at 158.242 104.902) (size 1.6) (drill 0.8) (layers F.Cu B.Cu) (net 30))
 (segment (start 155 107.14) (end 156.004 107.14) (width 0.7) (layer B.Cu) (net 30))
 (segment (start 156.004 107.14) (end 158.242 104.902) (width 0.7) (layer B.Cu) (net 30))
 (via (at 150.622 78.232) (size 1.6) (drill 0.8) (layers F.Cu B.Cu) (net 30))
 (segment (start 153.924 81.534) (end 153.924 92.202) (width 0.7) (layer F.Cu) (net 30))
 (segment (start 158.242 96.774) (end 158.242 104.902) (width 0.7) (layer F.Cu) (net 30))
 (segment (start 158.242 96.52) (end 158.242 96.774) (width 0.7) (layer F.Cu) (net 30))
 (segment (start 153.924 92.202) (end 158.242 96.52) (width 0.7) (layer F.Cu) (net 30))
 (segment (start 150.622 78.232) (end 153.924 81.534) (width 0.7) (layer F.Cu) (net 30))
 (segment (start 138.686 78.232) (end 138.606 78.312) (width 0.7) (layer B.Cu) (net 30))
 (segment (start 150.622 78.232) (end 138.686 78.232) (width 0.7) (layer B.Cu) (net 30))
 (segment (start 156.07763 109.68) (end 156.79163 108.966) (width 0.7) (layer B.Cu) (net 31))
 (segment (start 155 109.68) (end 156.07763 109.68) (width 0.7) (layer B.Cu) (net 31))
 (segment (start 156.79163 108.966) (end 157.988 108.966) (width 0.7) (layer B.Cu) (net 31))
 (segment (start 159.766 105.04063) (end 159.766 95.758) (width 0.7) (layer F.Cu) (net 31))
 (segment (start 159.766 95.758) (end 155.702 91.694) (width 0.7) (layer F.Cu) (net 31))
 (via (at 152.542 76.312) (size 1.6) (drill 0.8) (layers F.Cu B.Cu) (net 31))
 (segment (start 155.702 79.472) (end 152.542 76.312) (width 0.7) (layer F.Cu) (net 31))
 (segment (start 155.702 91.694) (end 155.702 79.472) (width 0.7) (layer F.Cu) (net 31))
 (segment (start 138.606 76.312) (end 152.542 76.312) (width 0.7) (layer B.Cu) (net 31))
 (via (at 159.004 107.95) (size 1.6) (drill 0.8) (layers F.Cu B.Cu) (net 31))
 (segment (start 157.988 108.966) (end 159.004 107.95) (width 0.7) (layer B.Cu) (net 31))
 (segment (start 159.004 106.81863) (end 159.766 106.05663) (width 0.7) (layer F.Cu) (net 31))
 (segment (start 159.766 106.05663) (end 159.766 105.04063) (width 0.7) (layer F.Cu) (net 31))
 (segment (start 159.004 107.95) (end 159.004 106.81863) (width 0.7) (layer F.Cu) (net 31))
 (segment (start 162.274 127.46) (end 162.306 127.428) (width 0.7) (layer B.Cu) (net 50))
 (segment (start 155 127.46) (end 162.274 127.46) (width 0.7) (layer B.Cu) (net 50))
 (segment (start 162.298 124.92) (end 162.306 124.928) (width 0.7) (layer B.Cu) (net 49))
 (segment (start 155 124.92) (end 162.298 124.92) (width 0.7) (layer B.Cu) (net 49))
 (segment (start 132.261 93.799) (end 132.334 93.726) (width 0.7) (layer B.Cu) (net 12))
 (segment (start 128.778 93.799) (end 132.261 93.799) (width 0.7) (layer B.Cu) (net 12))
 (via (at 152.4 122.174) (size 1.6) (drill 0.8) (layers F.Cu B.Cu) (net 1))
 (segment (start 149.606 122.228) (end 152.346 122.228) (width 0.7) (layer F.Cu) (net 1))
 (segment (start 152.346 122.228) (end 152.4 122.174) (width 0.7) (layer F.Cu) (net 1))
 (segment (start 154.794 122.174) (end 155 122.38) (width 0.7) (layer B.Cu) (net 1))
 (segment (start 152.4 122.174) (end 154.794 122.174) (width 0.7) (layer B.Cu) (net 1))
 (via (at 152.4 119.634) (size 1.6) (drill 0.8) (layers F.Cu B.Cu) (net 2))
 (segment (start 149.606 119.728) (end 152.306 119.728) (width 0.7) (layer F.Cu) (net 2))
 (segment (start 152.306 119.728) (end 152.4 119.634) (width 0.7) (layer F.Cu) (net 2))
 (segment (start 154.794 119.634) (end 155 119.84) (width 0.7) (layer B.Cu) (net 2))
 (segment (start 152.4 119.634) (end 154.794 119.634) (width 0.7) (layer B.Cu) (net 2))
 (segment (start 149.606 117.228) (end 152.28 117.228) (width 0.7) (layer F.Cu) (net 3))
 (via (at 152.4 117.348) (size 1.6) (drill 0.8) (layers F.Cu B.Cu) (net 3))
 (segment (start 152.28 117.228) (end 152.4 117.348) (width 0.7) (layer F.Cu) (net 3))
 (segment (start 154.952 117.348) (end 155 117.3) (width 0.7) (layer B.Cu) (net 3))
 (segment (start 152.4 117.348) (end 154.952 117.348) (width 0.7) (layer B.Cu) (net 3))
 (via (at 152.4 114.808) (size 1.6) (drill 0.8) (layers F.Cu B.Cu) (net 4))
 (segment (start 149.606 114.728) (end 152.32 114.728) (width 0.7) (layer F.Cu) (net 4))
 (segment (start 152.32 114.728) (end 152.4 114.808) (width 0.7) (layer F.Cu) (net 4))
 (segment (start 154.952 114.808) (end 155 114.76) (width 0.7) (layer B.Cu) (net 4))
 (segment (start 152.4 114.808) (end 154.952 114.808) (width 0.7) (layer B.Cu) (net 4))
 (via (at 152.4 112.268) (size 1.6) (drill 0.8) (layers F.Cu B.Cu) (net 5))
 (segment (start 149.606 112.228) (end 152.36 112.228) (width 0.7) (layer F.Cu) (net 5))
 (segment (start 152.36 112.228) (end 152.4 112.268) (width 0.7) (layer F.Cu) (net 5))
 (segment (start 154.952 112.268) (end 155 112.22) (width 0.7) (layer B.Cu) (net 5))
 (segment (start 152.4 112.268) (end 154.952 112.268) (width 0.7) (layer B.Cu) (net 5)))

